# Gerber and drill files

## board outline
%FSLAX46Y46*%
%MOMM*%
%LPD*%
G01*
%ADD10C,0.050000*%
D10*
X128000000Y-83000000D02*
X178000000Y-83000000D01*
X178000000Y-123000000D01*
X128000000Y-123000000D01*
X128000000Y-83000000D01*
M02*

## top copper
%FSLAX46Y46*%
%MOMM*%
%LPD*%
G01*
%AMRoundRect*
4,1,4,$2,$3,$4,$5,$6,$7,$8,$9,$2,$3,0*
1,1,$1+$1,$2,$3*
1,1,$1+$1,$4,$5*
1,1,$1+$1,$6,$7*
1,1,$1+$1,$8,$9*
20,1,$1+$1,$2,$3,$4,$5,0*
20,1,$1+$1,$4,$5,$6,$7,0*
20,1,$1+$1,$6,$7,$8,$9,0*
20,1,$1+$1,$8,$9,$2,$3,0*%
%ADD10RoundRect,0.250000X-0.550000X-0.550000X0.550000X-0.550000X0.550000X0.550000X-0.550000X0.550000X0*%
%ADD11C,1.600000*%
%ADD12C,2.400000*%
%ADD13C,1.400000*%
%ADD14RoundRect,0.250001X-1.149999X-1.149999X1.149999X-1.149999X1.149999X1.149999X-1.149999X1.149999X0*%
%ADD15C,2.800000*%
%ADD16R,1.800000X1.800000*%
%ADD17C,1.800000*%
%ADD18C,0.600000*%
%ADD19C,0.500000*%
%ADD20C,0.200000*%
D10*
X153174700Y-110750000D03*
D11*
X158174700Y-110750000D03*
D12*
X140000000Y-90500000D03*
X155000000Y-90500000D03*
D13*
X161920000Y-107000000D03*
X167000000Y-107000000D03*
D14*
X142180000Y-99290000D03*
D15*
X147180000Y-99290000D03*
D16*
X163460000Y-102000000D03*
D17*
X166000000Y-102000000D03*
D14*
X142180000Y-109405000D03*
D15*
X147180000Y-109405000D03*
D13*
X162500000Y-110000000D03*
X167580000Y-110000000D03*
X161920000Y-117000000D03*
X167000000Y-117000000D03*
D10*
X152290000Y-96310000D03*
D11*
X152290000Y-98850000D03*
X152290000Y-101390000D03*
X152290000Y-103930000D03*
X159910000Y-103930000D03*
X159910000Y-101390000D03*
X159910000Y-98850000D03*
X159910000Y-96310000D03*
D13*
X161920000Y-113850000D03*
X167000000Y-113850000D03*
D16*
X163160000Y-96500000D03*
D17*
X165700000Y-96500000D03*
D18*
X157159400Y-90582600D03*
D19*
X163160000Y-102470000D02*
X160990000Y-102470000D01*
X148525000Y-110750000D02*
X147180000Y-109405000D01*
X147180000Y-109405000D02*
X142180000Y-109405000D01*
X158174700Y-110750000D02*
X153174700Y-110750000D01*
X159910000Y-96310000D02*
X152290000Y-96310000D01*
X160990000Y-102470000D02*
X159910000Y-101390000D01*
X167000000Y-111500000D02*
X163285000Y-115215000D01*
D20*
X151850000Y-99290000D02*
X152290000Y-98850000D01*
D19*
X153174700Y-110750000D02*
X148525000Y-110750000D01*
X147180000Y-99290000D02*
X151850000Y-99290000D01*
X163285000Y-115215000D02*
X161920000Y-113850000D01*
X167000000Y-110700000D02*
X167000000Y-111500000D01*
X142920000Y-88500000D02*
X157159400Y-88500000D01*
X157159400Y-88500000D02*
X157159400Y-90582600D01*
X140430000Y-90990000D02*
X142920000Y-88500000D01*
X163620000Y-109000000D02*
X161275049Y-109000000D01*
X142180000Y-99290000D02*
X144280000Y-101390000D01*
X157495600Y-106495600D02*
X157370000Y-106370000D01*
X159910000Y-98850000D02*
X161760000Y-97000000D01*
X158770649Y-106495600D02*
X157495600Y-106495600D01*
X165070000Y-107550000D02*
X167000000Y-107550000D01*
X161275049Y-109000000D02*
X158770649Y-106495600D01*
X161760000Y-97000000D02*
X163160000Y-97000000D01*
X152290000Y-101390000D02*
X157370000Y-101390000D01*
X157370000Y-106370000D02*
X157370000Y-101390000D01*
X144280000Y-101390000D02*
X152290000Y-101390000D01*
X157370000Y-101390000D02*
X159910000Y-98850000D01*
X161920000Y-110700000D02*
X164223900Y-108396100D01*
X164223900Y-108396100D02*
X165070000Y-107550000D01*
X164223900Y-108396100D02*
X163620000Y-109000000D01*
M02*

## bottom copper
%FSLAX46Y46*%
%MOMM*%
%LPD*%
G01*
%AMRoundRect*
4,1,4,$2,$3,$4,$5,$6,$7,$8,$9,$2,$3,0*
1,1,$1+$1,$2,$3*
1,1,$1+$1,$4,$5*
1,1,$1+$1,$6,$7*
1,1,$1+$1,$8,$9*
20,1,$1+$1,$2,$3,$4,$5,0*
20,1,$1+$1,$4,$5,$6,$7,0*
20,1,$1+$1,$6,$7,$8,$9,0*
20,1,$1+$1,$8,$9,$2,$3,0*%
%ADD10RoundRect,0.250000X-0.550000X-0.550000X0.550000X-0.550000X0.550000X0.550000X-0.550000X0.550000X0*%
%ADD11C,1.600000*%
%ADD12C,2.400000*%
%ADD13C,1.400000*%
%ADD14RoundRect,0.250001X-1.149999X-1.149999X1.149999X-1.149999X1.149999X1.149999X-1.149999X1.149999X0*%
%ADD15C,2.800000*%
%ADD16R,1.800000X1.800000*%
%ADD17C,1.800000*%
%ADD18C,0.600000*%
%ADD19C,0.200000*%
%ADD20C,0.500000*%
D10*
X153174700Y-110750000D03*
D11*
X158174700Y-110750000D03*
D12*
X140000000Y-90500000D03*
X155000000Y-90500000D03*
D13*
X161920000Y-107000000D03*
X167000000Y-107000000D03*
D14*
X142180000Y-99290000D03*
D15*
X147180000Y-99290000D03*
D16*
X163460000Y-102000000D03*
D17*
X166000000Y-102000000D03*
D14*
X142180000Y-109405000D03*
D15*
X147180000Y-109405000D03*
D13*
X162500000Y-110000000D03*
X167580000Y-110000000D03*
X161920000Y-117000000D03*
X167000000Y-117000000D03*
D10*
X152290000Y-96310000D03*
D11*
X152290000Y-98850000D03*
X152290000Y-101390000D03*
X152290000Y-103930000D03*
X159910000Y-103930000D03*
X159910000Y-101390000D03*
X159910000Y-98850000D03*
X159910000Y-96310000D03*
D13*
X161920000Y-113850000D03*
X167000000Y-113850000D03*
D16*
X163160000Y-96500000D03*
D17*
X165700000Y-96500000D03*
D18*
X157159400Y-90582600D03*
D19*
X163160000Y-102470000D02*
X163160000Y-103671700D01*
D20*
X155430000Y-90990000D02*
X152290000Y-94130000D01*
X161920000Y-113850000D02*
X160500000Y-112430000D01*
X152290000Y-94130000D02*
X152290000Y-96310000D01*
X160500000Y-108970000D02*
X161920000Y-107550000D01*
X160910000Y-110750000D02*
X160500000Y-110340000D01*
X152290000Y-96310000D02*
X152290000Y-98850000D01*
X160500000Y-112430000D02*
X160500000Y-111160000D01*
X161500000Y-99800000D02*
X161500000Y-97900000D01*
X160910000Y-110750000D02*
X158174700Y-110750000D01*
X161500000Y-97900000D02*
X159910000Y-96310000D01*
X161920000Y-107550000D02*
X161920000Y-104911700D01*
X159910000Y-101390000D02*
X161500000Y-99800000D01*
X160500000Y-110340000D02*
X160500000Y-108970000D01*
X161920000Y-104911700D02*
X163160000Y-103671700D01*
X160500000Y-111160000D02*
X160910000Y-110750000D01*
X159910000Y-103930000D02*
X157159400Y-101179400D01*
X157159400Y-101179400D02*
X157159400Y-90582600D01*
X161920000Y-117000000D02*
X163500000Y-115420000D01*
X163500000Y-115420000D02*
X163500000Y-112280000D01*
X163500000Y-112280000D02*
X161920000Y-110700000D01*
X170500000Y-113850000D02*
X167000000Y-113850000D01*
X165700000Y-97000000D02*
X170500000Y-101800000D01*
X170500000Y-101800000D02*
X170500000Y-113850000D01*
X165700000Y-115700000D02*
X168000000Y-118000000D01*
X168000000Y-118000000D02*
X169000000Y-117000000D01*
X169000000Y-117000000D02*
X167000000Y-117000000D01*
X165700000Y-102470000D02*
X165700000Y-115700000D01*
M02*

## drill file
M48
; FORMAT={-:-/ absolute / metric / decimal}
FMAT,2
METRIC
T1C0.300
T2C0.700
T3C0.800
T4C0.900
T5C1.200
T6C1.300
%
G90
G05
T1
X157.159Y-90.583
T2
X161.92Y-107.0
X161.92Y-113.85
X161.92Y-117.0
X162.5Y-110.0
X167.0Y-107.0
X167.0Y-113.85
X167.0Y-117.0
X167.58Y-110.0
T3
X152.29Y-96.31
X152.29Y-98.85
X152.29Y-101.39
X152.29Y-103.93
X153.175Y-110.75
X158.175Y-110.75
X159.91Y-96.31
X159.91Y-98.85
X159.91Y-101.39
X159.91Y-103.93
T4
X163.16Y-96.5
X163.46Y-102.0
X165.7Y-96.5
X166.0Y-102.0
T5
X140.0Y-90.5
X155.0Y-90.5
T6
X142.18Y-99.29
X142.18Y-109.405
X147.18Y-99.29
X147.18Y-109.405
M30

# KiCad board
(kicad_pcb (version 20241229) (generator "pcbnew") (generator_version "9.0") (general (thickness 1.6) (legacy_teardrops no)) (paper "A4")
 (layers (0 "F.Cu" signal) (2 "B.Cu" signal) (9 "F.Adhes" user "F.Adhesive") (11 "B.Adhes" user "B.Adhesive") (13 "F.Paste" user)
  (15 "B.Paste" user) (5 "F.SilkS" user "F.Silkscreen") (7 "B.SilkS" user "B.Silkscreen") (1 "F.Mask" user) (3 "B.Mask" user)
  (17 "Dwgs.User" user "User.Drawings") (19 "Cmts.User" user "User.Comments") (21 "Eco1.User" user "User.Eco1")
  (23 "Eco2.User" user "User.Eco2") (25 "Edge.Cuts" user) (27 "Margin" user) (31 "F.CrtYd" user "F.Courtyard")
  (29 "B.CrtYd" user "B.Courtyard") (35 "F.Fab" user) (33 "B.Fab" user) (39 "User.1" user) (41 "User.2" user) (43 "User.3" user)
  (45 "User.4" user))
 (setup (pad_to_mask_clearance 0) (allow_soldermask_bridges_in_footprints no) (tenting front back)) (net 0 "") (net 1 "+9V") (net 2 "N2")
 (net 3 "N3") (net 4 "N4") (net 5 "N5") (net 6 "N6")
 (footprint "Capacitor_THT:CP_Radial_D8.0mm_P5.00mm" (layer "F.Cu") (at 153.1747 110.75)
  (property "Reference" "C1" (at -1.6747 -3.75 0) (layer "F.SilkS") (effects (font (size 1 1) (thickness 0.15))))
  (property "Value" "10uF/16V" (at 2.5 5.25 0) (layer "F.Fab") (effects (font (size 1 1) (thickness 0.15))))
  (pad "1" thru_hole roundrect (at 0 0) (size 1.6 1.6) (drill 0.8) (layers "*.Cu" "*.Mask") (remove_unused_layers no)
   (roundrect_rratio 0.15625) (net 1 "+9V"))
  (pad "2" thru_hole circle (at 5 0) (size 1.6 1.6) (drill 0.8) (layers "*.Cu" "*.Mask") (remove_unused_layers no) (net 1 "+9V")))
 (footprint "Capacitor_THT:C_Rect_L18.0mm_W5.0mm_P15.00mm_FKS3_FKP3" (layer "F.Cu") (at 140 90.5)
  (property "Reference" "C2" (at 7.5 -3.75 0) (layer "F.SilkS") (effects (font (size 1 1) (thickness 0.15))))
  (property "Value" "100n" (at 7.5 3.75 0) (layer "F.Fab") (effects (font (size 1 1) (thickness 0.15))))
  (pad "1" thru_hole circle (at 0 0) (size 2.4 2.4) (drill 1.2) (layers "*.Cu" "*.Mask") (remove_unused_layers no) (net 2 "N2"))
  (pad "2" thru_hole circle (at 15 0) (size 2.4 2.4) (drill 1.2) (layers "*.Cu" "*.Mask") (remove_unused_layers no) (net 1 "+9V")))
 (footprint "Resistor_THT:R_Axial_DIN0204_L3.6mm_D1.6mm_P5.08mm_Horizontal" (layer "F.Cu") (at 161.92 107)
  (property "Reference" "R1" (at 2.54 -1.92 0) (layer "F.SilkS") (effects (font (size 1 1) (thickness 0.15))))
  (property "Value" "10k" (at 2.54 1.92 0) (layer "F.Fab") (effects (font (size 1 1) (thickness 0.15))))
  (pad "1" thru_hole circle (at 0 0) (size 1.4 1.4) (drill 0.7) (layers "*.Cu" "*.Mask") (remove_unused_layers no) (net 1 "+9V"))
  (pad "2" thru_hole circle (at 5.08 0) (size 1.4 1.4) (drill 0.7) (layers "*.Cu" "*.Mask") (remove_unused_layers no) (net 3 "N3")))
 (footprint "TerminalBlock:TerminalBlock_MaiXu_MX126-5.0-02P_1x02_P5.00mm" (layer "F.Cu") (at 142.18 99.29)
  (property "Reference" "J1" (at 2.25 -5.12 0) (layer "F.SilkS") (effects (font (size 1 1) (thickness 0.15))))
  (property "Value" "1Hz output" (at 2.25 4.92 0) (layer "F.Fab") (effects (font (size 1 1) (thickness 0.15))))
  (pad "1" thru_hole roundrect (at 0 0) (size 2.8 2.8) (drill 1.3) (layers "*.Cu" "*.Mask") (remove_unused_layers no)
   (roundrect_rratio 0.089286) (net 3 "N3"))
  (pad "2" thru_hole circle (at 5 0) (size 2.8 2.8) (drill 1.3) (layers "*.Cu" "*.Mask") (remove_unused_layers no) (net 1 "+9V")))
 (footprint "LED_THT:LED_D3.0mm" (layer "F.Cu") (at 163.46 102)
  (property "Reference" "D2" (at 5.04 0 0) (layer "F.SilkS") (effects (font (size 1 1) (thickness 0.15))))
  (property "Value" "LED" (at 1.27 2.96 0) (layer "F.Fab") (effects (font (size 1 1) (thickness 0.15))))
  (pad "1" thru_hole rect (at 0 0) (size 1.8 1.8) (drill 0.9) (layers "*.Cu" "*.Mask") (remove_unused_layers no) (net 1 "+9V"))
  (pad "2" thru_hole circle (at 2.54 0) (size 1.8 1.8) (drill 0.9) (layers "*.Cu" "*.Mask") (remove_unused_layers no) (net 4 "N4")))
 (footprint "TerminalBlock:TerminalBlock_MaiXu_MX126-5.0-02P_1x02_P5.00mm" (layer "F.Cu") (at 142.18 109.405)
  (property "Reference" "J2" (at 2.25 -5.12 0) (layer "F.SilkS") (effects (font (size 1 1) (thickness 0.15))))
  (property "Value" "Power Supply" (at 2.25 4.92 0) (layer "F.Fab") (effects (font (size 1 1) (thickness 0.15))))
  (pad "1" thru_hole roundrect (at 0 0) (size 2.8 2.8) (drill 1.3) (layers "*.Cu" "*.Mask") (remove_unused_layers no)
   (roundrect_rratio 0.089286) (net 1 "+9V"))
  (pad "2" thru_hole circle (at 5 0) (size 2.8 2.8) (drill 1.3) (layers "*.Cu" "*.Mask") (remove_unused_layers no) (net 1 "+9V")))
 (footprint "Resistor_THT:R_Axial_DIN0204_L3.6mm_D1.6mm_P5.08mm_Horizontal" (layer "F.Cu") (at 162.5 110)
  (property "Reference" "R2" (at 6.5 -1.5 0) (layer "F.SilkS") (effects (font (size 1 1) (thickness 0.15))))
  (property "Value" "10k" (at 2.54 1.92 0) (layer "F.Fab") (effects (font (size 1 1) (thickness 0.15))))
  (pad "1" thru_hole circle (at 0 0) (size 1.4 1.4) (drill 0.7) (layers "*.Cu" "*.Mask") (remove_unused_layers no) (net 3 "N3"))
  (pad "2" thru_hole circle (at 5.08 0) (size 1.4 1.4) (drill 0.7) (layers "*.Cu" "*.Mask") (remove_unused_layers no) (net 1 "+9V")))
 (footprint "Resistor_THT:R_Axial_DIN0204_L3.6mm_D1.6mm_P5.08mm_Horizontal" (layer "F.Cu") (at 161.92 117)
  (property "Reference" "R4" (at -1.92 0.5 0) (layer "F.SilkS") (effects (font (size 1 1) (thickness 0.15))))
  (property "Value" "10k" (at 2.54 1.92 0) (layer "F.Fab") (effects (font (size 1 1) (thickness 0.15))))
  (pad "1" thru_hole circle (at 0 0) (size 1.4 1.4) (drill 0.7) (layers "*.Cu" "*.Mask") (remove_unused_layers no) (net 3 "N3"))
  (pad "2" thru_hole circle (at 5.08 0) (size 1.4 1.4) (drill 0.7) (layers "*.Cu" "*.Mask") (remove_unused_layers no) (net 4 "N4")))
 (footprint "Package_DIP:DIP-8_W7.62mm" (layer "F.Cu") (at 152.29 96.31)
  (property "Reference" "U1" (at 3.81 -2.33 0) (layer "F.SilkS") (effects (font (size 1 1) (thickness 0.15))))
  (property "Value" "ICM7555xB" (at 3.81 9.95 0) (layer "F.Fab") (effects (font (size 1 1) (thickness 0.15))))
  (pad "1" thru_hole roundrect (at 0 0) (size 1.6 1.6) (drill 0.8) (layers "*.Cu" "*.Mask") (remove_unused_layers no)
   (roundrect_rratio 0.15625) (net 1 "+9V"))
  (pad "2" thru_hole circle (at 0 2.54) (size 1.6 1.6) (drill 0.8) (layers "*.Cu" "*.Mask") (remove_unused_layers no) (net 1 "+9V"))
  (pad "3" thru_hole circle (at 0 5.08) (size 1.6 1.6) (drill 0.8) (layers "*.Cu" "*.Mask") (remove_unused_layers no) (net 3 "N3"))
  (pad "4" thru_hole circle (at 0 7.62) (size 1.6 1.6) (drill 0.8) (layers "*.Cu" "*.Mask") (remove_unused_layers no) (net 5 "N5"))
  (pad "5" thru_hole circle (at 7.62 7.62) (size 1.6 1.6) (drill 0.8) (layers "*.Cu" "*.Mask") (remove_unused_layers no) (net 2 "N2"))
  (pad "6" thru_hole circle (at 7.62 5.08) (size 1.6 1.6) (drill 0.8) (layers "*.Cu" "*.Mask") (remove_unused_layers no) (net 1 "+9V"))
  (pad "7" thru_hole circle (at 7.62 2.54) (size 1.6 1.6) (drill 0.8) (layers "*.Cu" "*.Mask") (remove_unused_layers no) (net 3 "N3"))
  (pad "8" thru_hole circle (at 7.62 0) (size 1.6 1.6) (drill 0.8) (layers "*.Cu" "*.Mask") (remove_unused_layers no) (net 1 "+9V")))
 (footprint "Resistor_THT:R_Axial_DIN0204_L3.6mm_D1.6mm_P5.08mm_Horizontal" (layer "F.Cu") (at 161.92 113.85)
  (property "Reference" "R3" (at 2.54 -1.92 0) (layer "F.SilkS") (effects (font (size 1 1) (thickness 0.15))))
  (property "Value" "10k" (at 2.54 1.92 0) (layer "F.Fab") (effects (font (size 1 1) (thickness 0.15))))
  (pad "1" thru_hole circle (at 0 0) (size 1.4 1.4) (drill 0.7) (layers "*.Cu" "*.Mask") (remove_unused_layers no) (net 1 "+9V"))
  (pad "2" thru_hole circle (at 5.08 0) (size 1.4 1.4) (drill 0.7) (layers "*.Cu" "*.Mask") (remove_unused_layers no) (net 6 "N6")))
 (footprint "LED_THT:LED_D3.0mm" (layer "F.Cu") (at 163.16 96.5)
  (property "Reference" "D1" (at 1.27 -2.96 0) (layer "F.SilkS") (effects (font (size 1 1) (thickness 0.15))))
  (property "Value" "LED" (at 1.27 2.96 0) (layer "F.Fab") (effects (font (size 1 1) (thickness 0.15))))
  (pad "1" thru_hole rect (at 0 0) (size 1.8 1.8) (drill 0.9) (layers "*.Cu" "*.Mask") (remove_unused_layers no) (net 3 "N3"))
  (pad "2" thru_hole circle (at 2.54 0) (size 1.8 1.8) (drill 0.9) (layers "*.Cu" "*.Mask") (remove_unused_layers no) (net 6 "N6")))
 (gr_rect (start 128 83) (end 178 123) (stroke (width 0.05) (type default)) (fill no) (layer "Edge.Cuts"))
 (segment (start 163.16 102.47) (end 160.99 102.47) (width 0.5) (layer "F.Cu") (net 1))
 (segment (start 148.525 110.75) (end 147.18 109.405) (width 0.5) (layer "F.Cu") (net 1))
 (segment (start 147.18 109.405) (end 142.18 109.405) (width 0.5) (layer "F.Cu") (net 1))
 (segment (start 158.1747 110.75) (end 153.1747 110.75) (width 0.5) (layer "F.Cu") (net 1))
 (segment (start 159.91 96.31) (end 152.29 96.31) (width 0.5) (layer "F.Cu") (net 1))
 (segment (start 160.99 102.47) (end 159.91 101.39) (width 0.5) (layer "F.Cu") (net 1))
 (segment (start 167 111.5) (end 163.285 115.215) (width 0.5) (layer "F.Cu") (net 1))
 (segment (start 151.85 99.29) (end 152.29 98.85) (width 0.2) (layer "F.Cu") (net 1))
 (segment (start 153.1747 110.75) (end 148.525 110.75) (width 0.5) (layer "F.Cu") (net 1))
 (segment (start 147.18 99.29) (end 151.85 99.29) (width 0.5) (layer "F.Cu") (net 1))
 (segment (start 163.285 115.215) (end 161.92 113.85) (width 0.5) (layer "F.Cu") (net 1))
 (segment (start 167 110.7) (end 167 111.5) (width 0.5) (layer "F.Cu") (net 1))
 (segment (start 163.16 102.47) (end 163.16 103.6717) (width 0.2) (layer "B.Cu") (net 1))
 (segment (start 155.43 90.99) (end 152.29 94.13) (width 0.5) (layer "B.Cu") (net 1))
 (segment (start 161.92 113.85) (end 160.5 112.43) (width 0.5) (layer "B.Cu") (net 1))
 (segment (start 152.29 94.13) (end 152.29 96.31) (width 0.5) (layer "B.Cu") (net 1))
 (segment (start 160.5 108.97) (end 161.92 107.55) (width 0.5) (layer "B.Cu") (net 1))
 (segment (start 160.91 110.75) (end 160.5 110.34) (width 0.5) (layer "B.Cu") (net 1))
 (segment (start 152.29 96.31) (end 152.29 98.85) (width 0.5) (layer "B.Cu") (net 1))
 (segment (start 160.5 112.43) (end 160.5 111.16) (width 0.5) (layer "B.Cu") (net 1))
 (segment (start 161.5 99.8) (end 161.5 97.9) (width 0.5) (layer "B.Cu") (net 1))
 (segment (start 160.91 110.75) (end 158.1747 110.75) (width 0.5) (layer "B.Cu") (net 1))
 (segment (start 161.5 97.9) (end 159.91 96.31) (width 0.5) (layer "B.Cu") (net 1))
 (segment (start 161.92 107.55) (end 161.92 104.9117) (width 0.5) (layer "B.Cu") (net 1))
 (segment (start 159.91 101.39) (end 161.5 99.8) (width 0.5) (layer "B.Cu") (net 1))
 (segment (start 160.5 110.34) (end 160.5 108.97) (width 0.5) (layer "B.Cu") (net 1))
 (segment (start 161.92 104.9117) (end 163.16 103.6717) (width 0.5) (layer "B.Cu") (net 1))
 (segment (start 160.5 111.16) (end 160.91 110.75) (width 0.5) (layer "B.Cu") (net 1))
 (segment (start 142.92 88.5) (end 157.1594 88.5) (width 0.5) (layer "F.Cu") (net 2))
 (segment (start 157.1594 88.5) (end 157.1594 90.5826) (width 0.5) (layer "F.Cu") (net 2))
 (segment (start 140.43 90.99) (end 142.92 88.5) (width 0.5) (layer "F.Cu") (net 2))
 (via (at 157.1594 90.5826) (size 0.6) (drill 0.3) (layers "F.Cu" "B.Cu") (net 2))
 (segment (start 159.91 103.93) (end 157.1594 101.1794) (width 0.5) (layer "B.Cu") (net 2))
 (segment (start 157.1594 101.1794) (end 157.1594 90.5826) (width 0.5) (layer "B.Cu") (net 2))
 (segment (start 163.62 109) (end 161.275049 109) (width 0.5) (layer "F.Cu") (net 3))
 (segment (start 142.18 99.29) (end 144.28 101.39) (width 0.5) (layer "F.Cu") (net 3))
 (segment (start 157.4956 106.4956) (end 157.37 106.37) (width 0.5) (layer "F.Cu") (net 3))
 (segment (start 159.91 98.85) (end 161.76 97) (width 0.5) (layer "F.Cu") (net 3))
 (segment (start 158.770649 106.4956) (end 157.4956 106.4956) (width 0.5) (layer "F.Cu") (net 3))
 (segment (start 165.07 107.55) (end 167 107.55) (width 0.5) (layer "F.Cu") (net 3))
 (segment (start 161.275049 109) (end 158.770649 106.4956) (width 0.5) (layer "F.Cu") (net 3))
 (segment (start 161.76 97) (end 163.16 97) (width 0.5) (layer "F.Cu") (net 3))
 (segment (start 152.29 101.39) (end 157.37 101.39) (width 0.5) (layer "F.Cu") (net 3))
 (segment (start 157.37 106.37) (end 157.37 101.39) (width 0.5) (layer "F.Cu") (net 3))
 (segment (start 144.28 101.39) (end 152.29 101.39) (width 0.5) (layer "F.Cu") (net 3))
 (segment (start 157.37 101.39) (end 159.91 98.85) (width 0.5) (layer "F.Cu") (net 3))
 (segment (start 161.92 110.7) (end 164.2239 108.3961) (width 0.5) (layer "F.Cu") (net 3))
 (segment (start 164.2239 108.3961) (end 165.07 107.55) (width 0.5) (layer "F.Cu") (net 3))
 (segment (start 164.2239 108.3961) (end 163.62 109) (width 0.5) (layer "F.Cu") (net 3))
 (segment (start 161.92 117) (end 163.5 115.42) (width 0.5) (layer "B.Cu") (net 3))
 (segment (start 163.5 115.42) (end 163.5 112.28) (width 0.5) (layer "B.Cu") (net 3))
 (segment (start 163.5 112.28) (end 161.92 110.7) (width 0.5) (layer "B.Cu") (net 3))
 (segment (start 170.5 113.85) (end 167 113.85) (width 0.5) (layer "B.Cu") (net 6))
 (segment (start 165.7 97) (end 170.5 101.8) (width 0.5) (layer "B.Cu") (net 6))
 (segment (start 170.5 101.8) (end 170.5 113.85) (width 0.5) (layer "B.Cu") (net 6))
 (segment (start 165.7 115.7) (end 168 118) (width 0.5) (layer "B.Cu") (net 4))
 (segment (start 168 118) (end 169 117) (width 0.5) (layer "B.Cu") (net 4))
 (segment (start 169 117) (end 167 117) (width 0.5) (layer "B.Cu") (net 4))
 (segment (start 165.7 102.47) (end 165.7 115.7) (width 0.5) (layer "B.Cu") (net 4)))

